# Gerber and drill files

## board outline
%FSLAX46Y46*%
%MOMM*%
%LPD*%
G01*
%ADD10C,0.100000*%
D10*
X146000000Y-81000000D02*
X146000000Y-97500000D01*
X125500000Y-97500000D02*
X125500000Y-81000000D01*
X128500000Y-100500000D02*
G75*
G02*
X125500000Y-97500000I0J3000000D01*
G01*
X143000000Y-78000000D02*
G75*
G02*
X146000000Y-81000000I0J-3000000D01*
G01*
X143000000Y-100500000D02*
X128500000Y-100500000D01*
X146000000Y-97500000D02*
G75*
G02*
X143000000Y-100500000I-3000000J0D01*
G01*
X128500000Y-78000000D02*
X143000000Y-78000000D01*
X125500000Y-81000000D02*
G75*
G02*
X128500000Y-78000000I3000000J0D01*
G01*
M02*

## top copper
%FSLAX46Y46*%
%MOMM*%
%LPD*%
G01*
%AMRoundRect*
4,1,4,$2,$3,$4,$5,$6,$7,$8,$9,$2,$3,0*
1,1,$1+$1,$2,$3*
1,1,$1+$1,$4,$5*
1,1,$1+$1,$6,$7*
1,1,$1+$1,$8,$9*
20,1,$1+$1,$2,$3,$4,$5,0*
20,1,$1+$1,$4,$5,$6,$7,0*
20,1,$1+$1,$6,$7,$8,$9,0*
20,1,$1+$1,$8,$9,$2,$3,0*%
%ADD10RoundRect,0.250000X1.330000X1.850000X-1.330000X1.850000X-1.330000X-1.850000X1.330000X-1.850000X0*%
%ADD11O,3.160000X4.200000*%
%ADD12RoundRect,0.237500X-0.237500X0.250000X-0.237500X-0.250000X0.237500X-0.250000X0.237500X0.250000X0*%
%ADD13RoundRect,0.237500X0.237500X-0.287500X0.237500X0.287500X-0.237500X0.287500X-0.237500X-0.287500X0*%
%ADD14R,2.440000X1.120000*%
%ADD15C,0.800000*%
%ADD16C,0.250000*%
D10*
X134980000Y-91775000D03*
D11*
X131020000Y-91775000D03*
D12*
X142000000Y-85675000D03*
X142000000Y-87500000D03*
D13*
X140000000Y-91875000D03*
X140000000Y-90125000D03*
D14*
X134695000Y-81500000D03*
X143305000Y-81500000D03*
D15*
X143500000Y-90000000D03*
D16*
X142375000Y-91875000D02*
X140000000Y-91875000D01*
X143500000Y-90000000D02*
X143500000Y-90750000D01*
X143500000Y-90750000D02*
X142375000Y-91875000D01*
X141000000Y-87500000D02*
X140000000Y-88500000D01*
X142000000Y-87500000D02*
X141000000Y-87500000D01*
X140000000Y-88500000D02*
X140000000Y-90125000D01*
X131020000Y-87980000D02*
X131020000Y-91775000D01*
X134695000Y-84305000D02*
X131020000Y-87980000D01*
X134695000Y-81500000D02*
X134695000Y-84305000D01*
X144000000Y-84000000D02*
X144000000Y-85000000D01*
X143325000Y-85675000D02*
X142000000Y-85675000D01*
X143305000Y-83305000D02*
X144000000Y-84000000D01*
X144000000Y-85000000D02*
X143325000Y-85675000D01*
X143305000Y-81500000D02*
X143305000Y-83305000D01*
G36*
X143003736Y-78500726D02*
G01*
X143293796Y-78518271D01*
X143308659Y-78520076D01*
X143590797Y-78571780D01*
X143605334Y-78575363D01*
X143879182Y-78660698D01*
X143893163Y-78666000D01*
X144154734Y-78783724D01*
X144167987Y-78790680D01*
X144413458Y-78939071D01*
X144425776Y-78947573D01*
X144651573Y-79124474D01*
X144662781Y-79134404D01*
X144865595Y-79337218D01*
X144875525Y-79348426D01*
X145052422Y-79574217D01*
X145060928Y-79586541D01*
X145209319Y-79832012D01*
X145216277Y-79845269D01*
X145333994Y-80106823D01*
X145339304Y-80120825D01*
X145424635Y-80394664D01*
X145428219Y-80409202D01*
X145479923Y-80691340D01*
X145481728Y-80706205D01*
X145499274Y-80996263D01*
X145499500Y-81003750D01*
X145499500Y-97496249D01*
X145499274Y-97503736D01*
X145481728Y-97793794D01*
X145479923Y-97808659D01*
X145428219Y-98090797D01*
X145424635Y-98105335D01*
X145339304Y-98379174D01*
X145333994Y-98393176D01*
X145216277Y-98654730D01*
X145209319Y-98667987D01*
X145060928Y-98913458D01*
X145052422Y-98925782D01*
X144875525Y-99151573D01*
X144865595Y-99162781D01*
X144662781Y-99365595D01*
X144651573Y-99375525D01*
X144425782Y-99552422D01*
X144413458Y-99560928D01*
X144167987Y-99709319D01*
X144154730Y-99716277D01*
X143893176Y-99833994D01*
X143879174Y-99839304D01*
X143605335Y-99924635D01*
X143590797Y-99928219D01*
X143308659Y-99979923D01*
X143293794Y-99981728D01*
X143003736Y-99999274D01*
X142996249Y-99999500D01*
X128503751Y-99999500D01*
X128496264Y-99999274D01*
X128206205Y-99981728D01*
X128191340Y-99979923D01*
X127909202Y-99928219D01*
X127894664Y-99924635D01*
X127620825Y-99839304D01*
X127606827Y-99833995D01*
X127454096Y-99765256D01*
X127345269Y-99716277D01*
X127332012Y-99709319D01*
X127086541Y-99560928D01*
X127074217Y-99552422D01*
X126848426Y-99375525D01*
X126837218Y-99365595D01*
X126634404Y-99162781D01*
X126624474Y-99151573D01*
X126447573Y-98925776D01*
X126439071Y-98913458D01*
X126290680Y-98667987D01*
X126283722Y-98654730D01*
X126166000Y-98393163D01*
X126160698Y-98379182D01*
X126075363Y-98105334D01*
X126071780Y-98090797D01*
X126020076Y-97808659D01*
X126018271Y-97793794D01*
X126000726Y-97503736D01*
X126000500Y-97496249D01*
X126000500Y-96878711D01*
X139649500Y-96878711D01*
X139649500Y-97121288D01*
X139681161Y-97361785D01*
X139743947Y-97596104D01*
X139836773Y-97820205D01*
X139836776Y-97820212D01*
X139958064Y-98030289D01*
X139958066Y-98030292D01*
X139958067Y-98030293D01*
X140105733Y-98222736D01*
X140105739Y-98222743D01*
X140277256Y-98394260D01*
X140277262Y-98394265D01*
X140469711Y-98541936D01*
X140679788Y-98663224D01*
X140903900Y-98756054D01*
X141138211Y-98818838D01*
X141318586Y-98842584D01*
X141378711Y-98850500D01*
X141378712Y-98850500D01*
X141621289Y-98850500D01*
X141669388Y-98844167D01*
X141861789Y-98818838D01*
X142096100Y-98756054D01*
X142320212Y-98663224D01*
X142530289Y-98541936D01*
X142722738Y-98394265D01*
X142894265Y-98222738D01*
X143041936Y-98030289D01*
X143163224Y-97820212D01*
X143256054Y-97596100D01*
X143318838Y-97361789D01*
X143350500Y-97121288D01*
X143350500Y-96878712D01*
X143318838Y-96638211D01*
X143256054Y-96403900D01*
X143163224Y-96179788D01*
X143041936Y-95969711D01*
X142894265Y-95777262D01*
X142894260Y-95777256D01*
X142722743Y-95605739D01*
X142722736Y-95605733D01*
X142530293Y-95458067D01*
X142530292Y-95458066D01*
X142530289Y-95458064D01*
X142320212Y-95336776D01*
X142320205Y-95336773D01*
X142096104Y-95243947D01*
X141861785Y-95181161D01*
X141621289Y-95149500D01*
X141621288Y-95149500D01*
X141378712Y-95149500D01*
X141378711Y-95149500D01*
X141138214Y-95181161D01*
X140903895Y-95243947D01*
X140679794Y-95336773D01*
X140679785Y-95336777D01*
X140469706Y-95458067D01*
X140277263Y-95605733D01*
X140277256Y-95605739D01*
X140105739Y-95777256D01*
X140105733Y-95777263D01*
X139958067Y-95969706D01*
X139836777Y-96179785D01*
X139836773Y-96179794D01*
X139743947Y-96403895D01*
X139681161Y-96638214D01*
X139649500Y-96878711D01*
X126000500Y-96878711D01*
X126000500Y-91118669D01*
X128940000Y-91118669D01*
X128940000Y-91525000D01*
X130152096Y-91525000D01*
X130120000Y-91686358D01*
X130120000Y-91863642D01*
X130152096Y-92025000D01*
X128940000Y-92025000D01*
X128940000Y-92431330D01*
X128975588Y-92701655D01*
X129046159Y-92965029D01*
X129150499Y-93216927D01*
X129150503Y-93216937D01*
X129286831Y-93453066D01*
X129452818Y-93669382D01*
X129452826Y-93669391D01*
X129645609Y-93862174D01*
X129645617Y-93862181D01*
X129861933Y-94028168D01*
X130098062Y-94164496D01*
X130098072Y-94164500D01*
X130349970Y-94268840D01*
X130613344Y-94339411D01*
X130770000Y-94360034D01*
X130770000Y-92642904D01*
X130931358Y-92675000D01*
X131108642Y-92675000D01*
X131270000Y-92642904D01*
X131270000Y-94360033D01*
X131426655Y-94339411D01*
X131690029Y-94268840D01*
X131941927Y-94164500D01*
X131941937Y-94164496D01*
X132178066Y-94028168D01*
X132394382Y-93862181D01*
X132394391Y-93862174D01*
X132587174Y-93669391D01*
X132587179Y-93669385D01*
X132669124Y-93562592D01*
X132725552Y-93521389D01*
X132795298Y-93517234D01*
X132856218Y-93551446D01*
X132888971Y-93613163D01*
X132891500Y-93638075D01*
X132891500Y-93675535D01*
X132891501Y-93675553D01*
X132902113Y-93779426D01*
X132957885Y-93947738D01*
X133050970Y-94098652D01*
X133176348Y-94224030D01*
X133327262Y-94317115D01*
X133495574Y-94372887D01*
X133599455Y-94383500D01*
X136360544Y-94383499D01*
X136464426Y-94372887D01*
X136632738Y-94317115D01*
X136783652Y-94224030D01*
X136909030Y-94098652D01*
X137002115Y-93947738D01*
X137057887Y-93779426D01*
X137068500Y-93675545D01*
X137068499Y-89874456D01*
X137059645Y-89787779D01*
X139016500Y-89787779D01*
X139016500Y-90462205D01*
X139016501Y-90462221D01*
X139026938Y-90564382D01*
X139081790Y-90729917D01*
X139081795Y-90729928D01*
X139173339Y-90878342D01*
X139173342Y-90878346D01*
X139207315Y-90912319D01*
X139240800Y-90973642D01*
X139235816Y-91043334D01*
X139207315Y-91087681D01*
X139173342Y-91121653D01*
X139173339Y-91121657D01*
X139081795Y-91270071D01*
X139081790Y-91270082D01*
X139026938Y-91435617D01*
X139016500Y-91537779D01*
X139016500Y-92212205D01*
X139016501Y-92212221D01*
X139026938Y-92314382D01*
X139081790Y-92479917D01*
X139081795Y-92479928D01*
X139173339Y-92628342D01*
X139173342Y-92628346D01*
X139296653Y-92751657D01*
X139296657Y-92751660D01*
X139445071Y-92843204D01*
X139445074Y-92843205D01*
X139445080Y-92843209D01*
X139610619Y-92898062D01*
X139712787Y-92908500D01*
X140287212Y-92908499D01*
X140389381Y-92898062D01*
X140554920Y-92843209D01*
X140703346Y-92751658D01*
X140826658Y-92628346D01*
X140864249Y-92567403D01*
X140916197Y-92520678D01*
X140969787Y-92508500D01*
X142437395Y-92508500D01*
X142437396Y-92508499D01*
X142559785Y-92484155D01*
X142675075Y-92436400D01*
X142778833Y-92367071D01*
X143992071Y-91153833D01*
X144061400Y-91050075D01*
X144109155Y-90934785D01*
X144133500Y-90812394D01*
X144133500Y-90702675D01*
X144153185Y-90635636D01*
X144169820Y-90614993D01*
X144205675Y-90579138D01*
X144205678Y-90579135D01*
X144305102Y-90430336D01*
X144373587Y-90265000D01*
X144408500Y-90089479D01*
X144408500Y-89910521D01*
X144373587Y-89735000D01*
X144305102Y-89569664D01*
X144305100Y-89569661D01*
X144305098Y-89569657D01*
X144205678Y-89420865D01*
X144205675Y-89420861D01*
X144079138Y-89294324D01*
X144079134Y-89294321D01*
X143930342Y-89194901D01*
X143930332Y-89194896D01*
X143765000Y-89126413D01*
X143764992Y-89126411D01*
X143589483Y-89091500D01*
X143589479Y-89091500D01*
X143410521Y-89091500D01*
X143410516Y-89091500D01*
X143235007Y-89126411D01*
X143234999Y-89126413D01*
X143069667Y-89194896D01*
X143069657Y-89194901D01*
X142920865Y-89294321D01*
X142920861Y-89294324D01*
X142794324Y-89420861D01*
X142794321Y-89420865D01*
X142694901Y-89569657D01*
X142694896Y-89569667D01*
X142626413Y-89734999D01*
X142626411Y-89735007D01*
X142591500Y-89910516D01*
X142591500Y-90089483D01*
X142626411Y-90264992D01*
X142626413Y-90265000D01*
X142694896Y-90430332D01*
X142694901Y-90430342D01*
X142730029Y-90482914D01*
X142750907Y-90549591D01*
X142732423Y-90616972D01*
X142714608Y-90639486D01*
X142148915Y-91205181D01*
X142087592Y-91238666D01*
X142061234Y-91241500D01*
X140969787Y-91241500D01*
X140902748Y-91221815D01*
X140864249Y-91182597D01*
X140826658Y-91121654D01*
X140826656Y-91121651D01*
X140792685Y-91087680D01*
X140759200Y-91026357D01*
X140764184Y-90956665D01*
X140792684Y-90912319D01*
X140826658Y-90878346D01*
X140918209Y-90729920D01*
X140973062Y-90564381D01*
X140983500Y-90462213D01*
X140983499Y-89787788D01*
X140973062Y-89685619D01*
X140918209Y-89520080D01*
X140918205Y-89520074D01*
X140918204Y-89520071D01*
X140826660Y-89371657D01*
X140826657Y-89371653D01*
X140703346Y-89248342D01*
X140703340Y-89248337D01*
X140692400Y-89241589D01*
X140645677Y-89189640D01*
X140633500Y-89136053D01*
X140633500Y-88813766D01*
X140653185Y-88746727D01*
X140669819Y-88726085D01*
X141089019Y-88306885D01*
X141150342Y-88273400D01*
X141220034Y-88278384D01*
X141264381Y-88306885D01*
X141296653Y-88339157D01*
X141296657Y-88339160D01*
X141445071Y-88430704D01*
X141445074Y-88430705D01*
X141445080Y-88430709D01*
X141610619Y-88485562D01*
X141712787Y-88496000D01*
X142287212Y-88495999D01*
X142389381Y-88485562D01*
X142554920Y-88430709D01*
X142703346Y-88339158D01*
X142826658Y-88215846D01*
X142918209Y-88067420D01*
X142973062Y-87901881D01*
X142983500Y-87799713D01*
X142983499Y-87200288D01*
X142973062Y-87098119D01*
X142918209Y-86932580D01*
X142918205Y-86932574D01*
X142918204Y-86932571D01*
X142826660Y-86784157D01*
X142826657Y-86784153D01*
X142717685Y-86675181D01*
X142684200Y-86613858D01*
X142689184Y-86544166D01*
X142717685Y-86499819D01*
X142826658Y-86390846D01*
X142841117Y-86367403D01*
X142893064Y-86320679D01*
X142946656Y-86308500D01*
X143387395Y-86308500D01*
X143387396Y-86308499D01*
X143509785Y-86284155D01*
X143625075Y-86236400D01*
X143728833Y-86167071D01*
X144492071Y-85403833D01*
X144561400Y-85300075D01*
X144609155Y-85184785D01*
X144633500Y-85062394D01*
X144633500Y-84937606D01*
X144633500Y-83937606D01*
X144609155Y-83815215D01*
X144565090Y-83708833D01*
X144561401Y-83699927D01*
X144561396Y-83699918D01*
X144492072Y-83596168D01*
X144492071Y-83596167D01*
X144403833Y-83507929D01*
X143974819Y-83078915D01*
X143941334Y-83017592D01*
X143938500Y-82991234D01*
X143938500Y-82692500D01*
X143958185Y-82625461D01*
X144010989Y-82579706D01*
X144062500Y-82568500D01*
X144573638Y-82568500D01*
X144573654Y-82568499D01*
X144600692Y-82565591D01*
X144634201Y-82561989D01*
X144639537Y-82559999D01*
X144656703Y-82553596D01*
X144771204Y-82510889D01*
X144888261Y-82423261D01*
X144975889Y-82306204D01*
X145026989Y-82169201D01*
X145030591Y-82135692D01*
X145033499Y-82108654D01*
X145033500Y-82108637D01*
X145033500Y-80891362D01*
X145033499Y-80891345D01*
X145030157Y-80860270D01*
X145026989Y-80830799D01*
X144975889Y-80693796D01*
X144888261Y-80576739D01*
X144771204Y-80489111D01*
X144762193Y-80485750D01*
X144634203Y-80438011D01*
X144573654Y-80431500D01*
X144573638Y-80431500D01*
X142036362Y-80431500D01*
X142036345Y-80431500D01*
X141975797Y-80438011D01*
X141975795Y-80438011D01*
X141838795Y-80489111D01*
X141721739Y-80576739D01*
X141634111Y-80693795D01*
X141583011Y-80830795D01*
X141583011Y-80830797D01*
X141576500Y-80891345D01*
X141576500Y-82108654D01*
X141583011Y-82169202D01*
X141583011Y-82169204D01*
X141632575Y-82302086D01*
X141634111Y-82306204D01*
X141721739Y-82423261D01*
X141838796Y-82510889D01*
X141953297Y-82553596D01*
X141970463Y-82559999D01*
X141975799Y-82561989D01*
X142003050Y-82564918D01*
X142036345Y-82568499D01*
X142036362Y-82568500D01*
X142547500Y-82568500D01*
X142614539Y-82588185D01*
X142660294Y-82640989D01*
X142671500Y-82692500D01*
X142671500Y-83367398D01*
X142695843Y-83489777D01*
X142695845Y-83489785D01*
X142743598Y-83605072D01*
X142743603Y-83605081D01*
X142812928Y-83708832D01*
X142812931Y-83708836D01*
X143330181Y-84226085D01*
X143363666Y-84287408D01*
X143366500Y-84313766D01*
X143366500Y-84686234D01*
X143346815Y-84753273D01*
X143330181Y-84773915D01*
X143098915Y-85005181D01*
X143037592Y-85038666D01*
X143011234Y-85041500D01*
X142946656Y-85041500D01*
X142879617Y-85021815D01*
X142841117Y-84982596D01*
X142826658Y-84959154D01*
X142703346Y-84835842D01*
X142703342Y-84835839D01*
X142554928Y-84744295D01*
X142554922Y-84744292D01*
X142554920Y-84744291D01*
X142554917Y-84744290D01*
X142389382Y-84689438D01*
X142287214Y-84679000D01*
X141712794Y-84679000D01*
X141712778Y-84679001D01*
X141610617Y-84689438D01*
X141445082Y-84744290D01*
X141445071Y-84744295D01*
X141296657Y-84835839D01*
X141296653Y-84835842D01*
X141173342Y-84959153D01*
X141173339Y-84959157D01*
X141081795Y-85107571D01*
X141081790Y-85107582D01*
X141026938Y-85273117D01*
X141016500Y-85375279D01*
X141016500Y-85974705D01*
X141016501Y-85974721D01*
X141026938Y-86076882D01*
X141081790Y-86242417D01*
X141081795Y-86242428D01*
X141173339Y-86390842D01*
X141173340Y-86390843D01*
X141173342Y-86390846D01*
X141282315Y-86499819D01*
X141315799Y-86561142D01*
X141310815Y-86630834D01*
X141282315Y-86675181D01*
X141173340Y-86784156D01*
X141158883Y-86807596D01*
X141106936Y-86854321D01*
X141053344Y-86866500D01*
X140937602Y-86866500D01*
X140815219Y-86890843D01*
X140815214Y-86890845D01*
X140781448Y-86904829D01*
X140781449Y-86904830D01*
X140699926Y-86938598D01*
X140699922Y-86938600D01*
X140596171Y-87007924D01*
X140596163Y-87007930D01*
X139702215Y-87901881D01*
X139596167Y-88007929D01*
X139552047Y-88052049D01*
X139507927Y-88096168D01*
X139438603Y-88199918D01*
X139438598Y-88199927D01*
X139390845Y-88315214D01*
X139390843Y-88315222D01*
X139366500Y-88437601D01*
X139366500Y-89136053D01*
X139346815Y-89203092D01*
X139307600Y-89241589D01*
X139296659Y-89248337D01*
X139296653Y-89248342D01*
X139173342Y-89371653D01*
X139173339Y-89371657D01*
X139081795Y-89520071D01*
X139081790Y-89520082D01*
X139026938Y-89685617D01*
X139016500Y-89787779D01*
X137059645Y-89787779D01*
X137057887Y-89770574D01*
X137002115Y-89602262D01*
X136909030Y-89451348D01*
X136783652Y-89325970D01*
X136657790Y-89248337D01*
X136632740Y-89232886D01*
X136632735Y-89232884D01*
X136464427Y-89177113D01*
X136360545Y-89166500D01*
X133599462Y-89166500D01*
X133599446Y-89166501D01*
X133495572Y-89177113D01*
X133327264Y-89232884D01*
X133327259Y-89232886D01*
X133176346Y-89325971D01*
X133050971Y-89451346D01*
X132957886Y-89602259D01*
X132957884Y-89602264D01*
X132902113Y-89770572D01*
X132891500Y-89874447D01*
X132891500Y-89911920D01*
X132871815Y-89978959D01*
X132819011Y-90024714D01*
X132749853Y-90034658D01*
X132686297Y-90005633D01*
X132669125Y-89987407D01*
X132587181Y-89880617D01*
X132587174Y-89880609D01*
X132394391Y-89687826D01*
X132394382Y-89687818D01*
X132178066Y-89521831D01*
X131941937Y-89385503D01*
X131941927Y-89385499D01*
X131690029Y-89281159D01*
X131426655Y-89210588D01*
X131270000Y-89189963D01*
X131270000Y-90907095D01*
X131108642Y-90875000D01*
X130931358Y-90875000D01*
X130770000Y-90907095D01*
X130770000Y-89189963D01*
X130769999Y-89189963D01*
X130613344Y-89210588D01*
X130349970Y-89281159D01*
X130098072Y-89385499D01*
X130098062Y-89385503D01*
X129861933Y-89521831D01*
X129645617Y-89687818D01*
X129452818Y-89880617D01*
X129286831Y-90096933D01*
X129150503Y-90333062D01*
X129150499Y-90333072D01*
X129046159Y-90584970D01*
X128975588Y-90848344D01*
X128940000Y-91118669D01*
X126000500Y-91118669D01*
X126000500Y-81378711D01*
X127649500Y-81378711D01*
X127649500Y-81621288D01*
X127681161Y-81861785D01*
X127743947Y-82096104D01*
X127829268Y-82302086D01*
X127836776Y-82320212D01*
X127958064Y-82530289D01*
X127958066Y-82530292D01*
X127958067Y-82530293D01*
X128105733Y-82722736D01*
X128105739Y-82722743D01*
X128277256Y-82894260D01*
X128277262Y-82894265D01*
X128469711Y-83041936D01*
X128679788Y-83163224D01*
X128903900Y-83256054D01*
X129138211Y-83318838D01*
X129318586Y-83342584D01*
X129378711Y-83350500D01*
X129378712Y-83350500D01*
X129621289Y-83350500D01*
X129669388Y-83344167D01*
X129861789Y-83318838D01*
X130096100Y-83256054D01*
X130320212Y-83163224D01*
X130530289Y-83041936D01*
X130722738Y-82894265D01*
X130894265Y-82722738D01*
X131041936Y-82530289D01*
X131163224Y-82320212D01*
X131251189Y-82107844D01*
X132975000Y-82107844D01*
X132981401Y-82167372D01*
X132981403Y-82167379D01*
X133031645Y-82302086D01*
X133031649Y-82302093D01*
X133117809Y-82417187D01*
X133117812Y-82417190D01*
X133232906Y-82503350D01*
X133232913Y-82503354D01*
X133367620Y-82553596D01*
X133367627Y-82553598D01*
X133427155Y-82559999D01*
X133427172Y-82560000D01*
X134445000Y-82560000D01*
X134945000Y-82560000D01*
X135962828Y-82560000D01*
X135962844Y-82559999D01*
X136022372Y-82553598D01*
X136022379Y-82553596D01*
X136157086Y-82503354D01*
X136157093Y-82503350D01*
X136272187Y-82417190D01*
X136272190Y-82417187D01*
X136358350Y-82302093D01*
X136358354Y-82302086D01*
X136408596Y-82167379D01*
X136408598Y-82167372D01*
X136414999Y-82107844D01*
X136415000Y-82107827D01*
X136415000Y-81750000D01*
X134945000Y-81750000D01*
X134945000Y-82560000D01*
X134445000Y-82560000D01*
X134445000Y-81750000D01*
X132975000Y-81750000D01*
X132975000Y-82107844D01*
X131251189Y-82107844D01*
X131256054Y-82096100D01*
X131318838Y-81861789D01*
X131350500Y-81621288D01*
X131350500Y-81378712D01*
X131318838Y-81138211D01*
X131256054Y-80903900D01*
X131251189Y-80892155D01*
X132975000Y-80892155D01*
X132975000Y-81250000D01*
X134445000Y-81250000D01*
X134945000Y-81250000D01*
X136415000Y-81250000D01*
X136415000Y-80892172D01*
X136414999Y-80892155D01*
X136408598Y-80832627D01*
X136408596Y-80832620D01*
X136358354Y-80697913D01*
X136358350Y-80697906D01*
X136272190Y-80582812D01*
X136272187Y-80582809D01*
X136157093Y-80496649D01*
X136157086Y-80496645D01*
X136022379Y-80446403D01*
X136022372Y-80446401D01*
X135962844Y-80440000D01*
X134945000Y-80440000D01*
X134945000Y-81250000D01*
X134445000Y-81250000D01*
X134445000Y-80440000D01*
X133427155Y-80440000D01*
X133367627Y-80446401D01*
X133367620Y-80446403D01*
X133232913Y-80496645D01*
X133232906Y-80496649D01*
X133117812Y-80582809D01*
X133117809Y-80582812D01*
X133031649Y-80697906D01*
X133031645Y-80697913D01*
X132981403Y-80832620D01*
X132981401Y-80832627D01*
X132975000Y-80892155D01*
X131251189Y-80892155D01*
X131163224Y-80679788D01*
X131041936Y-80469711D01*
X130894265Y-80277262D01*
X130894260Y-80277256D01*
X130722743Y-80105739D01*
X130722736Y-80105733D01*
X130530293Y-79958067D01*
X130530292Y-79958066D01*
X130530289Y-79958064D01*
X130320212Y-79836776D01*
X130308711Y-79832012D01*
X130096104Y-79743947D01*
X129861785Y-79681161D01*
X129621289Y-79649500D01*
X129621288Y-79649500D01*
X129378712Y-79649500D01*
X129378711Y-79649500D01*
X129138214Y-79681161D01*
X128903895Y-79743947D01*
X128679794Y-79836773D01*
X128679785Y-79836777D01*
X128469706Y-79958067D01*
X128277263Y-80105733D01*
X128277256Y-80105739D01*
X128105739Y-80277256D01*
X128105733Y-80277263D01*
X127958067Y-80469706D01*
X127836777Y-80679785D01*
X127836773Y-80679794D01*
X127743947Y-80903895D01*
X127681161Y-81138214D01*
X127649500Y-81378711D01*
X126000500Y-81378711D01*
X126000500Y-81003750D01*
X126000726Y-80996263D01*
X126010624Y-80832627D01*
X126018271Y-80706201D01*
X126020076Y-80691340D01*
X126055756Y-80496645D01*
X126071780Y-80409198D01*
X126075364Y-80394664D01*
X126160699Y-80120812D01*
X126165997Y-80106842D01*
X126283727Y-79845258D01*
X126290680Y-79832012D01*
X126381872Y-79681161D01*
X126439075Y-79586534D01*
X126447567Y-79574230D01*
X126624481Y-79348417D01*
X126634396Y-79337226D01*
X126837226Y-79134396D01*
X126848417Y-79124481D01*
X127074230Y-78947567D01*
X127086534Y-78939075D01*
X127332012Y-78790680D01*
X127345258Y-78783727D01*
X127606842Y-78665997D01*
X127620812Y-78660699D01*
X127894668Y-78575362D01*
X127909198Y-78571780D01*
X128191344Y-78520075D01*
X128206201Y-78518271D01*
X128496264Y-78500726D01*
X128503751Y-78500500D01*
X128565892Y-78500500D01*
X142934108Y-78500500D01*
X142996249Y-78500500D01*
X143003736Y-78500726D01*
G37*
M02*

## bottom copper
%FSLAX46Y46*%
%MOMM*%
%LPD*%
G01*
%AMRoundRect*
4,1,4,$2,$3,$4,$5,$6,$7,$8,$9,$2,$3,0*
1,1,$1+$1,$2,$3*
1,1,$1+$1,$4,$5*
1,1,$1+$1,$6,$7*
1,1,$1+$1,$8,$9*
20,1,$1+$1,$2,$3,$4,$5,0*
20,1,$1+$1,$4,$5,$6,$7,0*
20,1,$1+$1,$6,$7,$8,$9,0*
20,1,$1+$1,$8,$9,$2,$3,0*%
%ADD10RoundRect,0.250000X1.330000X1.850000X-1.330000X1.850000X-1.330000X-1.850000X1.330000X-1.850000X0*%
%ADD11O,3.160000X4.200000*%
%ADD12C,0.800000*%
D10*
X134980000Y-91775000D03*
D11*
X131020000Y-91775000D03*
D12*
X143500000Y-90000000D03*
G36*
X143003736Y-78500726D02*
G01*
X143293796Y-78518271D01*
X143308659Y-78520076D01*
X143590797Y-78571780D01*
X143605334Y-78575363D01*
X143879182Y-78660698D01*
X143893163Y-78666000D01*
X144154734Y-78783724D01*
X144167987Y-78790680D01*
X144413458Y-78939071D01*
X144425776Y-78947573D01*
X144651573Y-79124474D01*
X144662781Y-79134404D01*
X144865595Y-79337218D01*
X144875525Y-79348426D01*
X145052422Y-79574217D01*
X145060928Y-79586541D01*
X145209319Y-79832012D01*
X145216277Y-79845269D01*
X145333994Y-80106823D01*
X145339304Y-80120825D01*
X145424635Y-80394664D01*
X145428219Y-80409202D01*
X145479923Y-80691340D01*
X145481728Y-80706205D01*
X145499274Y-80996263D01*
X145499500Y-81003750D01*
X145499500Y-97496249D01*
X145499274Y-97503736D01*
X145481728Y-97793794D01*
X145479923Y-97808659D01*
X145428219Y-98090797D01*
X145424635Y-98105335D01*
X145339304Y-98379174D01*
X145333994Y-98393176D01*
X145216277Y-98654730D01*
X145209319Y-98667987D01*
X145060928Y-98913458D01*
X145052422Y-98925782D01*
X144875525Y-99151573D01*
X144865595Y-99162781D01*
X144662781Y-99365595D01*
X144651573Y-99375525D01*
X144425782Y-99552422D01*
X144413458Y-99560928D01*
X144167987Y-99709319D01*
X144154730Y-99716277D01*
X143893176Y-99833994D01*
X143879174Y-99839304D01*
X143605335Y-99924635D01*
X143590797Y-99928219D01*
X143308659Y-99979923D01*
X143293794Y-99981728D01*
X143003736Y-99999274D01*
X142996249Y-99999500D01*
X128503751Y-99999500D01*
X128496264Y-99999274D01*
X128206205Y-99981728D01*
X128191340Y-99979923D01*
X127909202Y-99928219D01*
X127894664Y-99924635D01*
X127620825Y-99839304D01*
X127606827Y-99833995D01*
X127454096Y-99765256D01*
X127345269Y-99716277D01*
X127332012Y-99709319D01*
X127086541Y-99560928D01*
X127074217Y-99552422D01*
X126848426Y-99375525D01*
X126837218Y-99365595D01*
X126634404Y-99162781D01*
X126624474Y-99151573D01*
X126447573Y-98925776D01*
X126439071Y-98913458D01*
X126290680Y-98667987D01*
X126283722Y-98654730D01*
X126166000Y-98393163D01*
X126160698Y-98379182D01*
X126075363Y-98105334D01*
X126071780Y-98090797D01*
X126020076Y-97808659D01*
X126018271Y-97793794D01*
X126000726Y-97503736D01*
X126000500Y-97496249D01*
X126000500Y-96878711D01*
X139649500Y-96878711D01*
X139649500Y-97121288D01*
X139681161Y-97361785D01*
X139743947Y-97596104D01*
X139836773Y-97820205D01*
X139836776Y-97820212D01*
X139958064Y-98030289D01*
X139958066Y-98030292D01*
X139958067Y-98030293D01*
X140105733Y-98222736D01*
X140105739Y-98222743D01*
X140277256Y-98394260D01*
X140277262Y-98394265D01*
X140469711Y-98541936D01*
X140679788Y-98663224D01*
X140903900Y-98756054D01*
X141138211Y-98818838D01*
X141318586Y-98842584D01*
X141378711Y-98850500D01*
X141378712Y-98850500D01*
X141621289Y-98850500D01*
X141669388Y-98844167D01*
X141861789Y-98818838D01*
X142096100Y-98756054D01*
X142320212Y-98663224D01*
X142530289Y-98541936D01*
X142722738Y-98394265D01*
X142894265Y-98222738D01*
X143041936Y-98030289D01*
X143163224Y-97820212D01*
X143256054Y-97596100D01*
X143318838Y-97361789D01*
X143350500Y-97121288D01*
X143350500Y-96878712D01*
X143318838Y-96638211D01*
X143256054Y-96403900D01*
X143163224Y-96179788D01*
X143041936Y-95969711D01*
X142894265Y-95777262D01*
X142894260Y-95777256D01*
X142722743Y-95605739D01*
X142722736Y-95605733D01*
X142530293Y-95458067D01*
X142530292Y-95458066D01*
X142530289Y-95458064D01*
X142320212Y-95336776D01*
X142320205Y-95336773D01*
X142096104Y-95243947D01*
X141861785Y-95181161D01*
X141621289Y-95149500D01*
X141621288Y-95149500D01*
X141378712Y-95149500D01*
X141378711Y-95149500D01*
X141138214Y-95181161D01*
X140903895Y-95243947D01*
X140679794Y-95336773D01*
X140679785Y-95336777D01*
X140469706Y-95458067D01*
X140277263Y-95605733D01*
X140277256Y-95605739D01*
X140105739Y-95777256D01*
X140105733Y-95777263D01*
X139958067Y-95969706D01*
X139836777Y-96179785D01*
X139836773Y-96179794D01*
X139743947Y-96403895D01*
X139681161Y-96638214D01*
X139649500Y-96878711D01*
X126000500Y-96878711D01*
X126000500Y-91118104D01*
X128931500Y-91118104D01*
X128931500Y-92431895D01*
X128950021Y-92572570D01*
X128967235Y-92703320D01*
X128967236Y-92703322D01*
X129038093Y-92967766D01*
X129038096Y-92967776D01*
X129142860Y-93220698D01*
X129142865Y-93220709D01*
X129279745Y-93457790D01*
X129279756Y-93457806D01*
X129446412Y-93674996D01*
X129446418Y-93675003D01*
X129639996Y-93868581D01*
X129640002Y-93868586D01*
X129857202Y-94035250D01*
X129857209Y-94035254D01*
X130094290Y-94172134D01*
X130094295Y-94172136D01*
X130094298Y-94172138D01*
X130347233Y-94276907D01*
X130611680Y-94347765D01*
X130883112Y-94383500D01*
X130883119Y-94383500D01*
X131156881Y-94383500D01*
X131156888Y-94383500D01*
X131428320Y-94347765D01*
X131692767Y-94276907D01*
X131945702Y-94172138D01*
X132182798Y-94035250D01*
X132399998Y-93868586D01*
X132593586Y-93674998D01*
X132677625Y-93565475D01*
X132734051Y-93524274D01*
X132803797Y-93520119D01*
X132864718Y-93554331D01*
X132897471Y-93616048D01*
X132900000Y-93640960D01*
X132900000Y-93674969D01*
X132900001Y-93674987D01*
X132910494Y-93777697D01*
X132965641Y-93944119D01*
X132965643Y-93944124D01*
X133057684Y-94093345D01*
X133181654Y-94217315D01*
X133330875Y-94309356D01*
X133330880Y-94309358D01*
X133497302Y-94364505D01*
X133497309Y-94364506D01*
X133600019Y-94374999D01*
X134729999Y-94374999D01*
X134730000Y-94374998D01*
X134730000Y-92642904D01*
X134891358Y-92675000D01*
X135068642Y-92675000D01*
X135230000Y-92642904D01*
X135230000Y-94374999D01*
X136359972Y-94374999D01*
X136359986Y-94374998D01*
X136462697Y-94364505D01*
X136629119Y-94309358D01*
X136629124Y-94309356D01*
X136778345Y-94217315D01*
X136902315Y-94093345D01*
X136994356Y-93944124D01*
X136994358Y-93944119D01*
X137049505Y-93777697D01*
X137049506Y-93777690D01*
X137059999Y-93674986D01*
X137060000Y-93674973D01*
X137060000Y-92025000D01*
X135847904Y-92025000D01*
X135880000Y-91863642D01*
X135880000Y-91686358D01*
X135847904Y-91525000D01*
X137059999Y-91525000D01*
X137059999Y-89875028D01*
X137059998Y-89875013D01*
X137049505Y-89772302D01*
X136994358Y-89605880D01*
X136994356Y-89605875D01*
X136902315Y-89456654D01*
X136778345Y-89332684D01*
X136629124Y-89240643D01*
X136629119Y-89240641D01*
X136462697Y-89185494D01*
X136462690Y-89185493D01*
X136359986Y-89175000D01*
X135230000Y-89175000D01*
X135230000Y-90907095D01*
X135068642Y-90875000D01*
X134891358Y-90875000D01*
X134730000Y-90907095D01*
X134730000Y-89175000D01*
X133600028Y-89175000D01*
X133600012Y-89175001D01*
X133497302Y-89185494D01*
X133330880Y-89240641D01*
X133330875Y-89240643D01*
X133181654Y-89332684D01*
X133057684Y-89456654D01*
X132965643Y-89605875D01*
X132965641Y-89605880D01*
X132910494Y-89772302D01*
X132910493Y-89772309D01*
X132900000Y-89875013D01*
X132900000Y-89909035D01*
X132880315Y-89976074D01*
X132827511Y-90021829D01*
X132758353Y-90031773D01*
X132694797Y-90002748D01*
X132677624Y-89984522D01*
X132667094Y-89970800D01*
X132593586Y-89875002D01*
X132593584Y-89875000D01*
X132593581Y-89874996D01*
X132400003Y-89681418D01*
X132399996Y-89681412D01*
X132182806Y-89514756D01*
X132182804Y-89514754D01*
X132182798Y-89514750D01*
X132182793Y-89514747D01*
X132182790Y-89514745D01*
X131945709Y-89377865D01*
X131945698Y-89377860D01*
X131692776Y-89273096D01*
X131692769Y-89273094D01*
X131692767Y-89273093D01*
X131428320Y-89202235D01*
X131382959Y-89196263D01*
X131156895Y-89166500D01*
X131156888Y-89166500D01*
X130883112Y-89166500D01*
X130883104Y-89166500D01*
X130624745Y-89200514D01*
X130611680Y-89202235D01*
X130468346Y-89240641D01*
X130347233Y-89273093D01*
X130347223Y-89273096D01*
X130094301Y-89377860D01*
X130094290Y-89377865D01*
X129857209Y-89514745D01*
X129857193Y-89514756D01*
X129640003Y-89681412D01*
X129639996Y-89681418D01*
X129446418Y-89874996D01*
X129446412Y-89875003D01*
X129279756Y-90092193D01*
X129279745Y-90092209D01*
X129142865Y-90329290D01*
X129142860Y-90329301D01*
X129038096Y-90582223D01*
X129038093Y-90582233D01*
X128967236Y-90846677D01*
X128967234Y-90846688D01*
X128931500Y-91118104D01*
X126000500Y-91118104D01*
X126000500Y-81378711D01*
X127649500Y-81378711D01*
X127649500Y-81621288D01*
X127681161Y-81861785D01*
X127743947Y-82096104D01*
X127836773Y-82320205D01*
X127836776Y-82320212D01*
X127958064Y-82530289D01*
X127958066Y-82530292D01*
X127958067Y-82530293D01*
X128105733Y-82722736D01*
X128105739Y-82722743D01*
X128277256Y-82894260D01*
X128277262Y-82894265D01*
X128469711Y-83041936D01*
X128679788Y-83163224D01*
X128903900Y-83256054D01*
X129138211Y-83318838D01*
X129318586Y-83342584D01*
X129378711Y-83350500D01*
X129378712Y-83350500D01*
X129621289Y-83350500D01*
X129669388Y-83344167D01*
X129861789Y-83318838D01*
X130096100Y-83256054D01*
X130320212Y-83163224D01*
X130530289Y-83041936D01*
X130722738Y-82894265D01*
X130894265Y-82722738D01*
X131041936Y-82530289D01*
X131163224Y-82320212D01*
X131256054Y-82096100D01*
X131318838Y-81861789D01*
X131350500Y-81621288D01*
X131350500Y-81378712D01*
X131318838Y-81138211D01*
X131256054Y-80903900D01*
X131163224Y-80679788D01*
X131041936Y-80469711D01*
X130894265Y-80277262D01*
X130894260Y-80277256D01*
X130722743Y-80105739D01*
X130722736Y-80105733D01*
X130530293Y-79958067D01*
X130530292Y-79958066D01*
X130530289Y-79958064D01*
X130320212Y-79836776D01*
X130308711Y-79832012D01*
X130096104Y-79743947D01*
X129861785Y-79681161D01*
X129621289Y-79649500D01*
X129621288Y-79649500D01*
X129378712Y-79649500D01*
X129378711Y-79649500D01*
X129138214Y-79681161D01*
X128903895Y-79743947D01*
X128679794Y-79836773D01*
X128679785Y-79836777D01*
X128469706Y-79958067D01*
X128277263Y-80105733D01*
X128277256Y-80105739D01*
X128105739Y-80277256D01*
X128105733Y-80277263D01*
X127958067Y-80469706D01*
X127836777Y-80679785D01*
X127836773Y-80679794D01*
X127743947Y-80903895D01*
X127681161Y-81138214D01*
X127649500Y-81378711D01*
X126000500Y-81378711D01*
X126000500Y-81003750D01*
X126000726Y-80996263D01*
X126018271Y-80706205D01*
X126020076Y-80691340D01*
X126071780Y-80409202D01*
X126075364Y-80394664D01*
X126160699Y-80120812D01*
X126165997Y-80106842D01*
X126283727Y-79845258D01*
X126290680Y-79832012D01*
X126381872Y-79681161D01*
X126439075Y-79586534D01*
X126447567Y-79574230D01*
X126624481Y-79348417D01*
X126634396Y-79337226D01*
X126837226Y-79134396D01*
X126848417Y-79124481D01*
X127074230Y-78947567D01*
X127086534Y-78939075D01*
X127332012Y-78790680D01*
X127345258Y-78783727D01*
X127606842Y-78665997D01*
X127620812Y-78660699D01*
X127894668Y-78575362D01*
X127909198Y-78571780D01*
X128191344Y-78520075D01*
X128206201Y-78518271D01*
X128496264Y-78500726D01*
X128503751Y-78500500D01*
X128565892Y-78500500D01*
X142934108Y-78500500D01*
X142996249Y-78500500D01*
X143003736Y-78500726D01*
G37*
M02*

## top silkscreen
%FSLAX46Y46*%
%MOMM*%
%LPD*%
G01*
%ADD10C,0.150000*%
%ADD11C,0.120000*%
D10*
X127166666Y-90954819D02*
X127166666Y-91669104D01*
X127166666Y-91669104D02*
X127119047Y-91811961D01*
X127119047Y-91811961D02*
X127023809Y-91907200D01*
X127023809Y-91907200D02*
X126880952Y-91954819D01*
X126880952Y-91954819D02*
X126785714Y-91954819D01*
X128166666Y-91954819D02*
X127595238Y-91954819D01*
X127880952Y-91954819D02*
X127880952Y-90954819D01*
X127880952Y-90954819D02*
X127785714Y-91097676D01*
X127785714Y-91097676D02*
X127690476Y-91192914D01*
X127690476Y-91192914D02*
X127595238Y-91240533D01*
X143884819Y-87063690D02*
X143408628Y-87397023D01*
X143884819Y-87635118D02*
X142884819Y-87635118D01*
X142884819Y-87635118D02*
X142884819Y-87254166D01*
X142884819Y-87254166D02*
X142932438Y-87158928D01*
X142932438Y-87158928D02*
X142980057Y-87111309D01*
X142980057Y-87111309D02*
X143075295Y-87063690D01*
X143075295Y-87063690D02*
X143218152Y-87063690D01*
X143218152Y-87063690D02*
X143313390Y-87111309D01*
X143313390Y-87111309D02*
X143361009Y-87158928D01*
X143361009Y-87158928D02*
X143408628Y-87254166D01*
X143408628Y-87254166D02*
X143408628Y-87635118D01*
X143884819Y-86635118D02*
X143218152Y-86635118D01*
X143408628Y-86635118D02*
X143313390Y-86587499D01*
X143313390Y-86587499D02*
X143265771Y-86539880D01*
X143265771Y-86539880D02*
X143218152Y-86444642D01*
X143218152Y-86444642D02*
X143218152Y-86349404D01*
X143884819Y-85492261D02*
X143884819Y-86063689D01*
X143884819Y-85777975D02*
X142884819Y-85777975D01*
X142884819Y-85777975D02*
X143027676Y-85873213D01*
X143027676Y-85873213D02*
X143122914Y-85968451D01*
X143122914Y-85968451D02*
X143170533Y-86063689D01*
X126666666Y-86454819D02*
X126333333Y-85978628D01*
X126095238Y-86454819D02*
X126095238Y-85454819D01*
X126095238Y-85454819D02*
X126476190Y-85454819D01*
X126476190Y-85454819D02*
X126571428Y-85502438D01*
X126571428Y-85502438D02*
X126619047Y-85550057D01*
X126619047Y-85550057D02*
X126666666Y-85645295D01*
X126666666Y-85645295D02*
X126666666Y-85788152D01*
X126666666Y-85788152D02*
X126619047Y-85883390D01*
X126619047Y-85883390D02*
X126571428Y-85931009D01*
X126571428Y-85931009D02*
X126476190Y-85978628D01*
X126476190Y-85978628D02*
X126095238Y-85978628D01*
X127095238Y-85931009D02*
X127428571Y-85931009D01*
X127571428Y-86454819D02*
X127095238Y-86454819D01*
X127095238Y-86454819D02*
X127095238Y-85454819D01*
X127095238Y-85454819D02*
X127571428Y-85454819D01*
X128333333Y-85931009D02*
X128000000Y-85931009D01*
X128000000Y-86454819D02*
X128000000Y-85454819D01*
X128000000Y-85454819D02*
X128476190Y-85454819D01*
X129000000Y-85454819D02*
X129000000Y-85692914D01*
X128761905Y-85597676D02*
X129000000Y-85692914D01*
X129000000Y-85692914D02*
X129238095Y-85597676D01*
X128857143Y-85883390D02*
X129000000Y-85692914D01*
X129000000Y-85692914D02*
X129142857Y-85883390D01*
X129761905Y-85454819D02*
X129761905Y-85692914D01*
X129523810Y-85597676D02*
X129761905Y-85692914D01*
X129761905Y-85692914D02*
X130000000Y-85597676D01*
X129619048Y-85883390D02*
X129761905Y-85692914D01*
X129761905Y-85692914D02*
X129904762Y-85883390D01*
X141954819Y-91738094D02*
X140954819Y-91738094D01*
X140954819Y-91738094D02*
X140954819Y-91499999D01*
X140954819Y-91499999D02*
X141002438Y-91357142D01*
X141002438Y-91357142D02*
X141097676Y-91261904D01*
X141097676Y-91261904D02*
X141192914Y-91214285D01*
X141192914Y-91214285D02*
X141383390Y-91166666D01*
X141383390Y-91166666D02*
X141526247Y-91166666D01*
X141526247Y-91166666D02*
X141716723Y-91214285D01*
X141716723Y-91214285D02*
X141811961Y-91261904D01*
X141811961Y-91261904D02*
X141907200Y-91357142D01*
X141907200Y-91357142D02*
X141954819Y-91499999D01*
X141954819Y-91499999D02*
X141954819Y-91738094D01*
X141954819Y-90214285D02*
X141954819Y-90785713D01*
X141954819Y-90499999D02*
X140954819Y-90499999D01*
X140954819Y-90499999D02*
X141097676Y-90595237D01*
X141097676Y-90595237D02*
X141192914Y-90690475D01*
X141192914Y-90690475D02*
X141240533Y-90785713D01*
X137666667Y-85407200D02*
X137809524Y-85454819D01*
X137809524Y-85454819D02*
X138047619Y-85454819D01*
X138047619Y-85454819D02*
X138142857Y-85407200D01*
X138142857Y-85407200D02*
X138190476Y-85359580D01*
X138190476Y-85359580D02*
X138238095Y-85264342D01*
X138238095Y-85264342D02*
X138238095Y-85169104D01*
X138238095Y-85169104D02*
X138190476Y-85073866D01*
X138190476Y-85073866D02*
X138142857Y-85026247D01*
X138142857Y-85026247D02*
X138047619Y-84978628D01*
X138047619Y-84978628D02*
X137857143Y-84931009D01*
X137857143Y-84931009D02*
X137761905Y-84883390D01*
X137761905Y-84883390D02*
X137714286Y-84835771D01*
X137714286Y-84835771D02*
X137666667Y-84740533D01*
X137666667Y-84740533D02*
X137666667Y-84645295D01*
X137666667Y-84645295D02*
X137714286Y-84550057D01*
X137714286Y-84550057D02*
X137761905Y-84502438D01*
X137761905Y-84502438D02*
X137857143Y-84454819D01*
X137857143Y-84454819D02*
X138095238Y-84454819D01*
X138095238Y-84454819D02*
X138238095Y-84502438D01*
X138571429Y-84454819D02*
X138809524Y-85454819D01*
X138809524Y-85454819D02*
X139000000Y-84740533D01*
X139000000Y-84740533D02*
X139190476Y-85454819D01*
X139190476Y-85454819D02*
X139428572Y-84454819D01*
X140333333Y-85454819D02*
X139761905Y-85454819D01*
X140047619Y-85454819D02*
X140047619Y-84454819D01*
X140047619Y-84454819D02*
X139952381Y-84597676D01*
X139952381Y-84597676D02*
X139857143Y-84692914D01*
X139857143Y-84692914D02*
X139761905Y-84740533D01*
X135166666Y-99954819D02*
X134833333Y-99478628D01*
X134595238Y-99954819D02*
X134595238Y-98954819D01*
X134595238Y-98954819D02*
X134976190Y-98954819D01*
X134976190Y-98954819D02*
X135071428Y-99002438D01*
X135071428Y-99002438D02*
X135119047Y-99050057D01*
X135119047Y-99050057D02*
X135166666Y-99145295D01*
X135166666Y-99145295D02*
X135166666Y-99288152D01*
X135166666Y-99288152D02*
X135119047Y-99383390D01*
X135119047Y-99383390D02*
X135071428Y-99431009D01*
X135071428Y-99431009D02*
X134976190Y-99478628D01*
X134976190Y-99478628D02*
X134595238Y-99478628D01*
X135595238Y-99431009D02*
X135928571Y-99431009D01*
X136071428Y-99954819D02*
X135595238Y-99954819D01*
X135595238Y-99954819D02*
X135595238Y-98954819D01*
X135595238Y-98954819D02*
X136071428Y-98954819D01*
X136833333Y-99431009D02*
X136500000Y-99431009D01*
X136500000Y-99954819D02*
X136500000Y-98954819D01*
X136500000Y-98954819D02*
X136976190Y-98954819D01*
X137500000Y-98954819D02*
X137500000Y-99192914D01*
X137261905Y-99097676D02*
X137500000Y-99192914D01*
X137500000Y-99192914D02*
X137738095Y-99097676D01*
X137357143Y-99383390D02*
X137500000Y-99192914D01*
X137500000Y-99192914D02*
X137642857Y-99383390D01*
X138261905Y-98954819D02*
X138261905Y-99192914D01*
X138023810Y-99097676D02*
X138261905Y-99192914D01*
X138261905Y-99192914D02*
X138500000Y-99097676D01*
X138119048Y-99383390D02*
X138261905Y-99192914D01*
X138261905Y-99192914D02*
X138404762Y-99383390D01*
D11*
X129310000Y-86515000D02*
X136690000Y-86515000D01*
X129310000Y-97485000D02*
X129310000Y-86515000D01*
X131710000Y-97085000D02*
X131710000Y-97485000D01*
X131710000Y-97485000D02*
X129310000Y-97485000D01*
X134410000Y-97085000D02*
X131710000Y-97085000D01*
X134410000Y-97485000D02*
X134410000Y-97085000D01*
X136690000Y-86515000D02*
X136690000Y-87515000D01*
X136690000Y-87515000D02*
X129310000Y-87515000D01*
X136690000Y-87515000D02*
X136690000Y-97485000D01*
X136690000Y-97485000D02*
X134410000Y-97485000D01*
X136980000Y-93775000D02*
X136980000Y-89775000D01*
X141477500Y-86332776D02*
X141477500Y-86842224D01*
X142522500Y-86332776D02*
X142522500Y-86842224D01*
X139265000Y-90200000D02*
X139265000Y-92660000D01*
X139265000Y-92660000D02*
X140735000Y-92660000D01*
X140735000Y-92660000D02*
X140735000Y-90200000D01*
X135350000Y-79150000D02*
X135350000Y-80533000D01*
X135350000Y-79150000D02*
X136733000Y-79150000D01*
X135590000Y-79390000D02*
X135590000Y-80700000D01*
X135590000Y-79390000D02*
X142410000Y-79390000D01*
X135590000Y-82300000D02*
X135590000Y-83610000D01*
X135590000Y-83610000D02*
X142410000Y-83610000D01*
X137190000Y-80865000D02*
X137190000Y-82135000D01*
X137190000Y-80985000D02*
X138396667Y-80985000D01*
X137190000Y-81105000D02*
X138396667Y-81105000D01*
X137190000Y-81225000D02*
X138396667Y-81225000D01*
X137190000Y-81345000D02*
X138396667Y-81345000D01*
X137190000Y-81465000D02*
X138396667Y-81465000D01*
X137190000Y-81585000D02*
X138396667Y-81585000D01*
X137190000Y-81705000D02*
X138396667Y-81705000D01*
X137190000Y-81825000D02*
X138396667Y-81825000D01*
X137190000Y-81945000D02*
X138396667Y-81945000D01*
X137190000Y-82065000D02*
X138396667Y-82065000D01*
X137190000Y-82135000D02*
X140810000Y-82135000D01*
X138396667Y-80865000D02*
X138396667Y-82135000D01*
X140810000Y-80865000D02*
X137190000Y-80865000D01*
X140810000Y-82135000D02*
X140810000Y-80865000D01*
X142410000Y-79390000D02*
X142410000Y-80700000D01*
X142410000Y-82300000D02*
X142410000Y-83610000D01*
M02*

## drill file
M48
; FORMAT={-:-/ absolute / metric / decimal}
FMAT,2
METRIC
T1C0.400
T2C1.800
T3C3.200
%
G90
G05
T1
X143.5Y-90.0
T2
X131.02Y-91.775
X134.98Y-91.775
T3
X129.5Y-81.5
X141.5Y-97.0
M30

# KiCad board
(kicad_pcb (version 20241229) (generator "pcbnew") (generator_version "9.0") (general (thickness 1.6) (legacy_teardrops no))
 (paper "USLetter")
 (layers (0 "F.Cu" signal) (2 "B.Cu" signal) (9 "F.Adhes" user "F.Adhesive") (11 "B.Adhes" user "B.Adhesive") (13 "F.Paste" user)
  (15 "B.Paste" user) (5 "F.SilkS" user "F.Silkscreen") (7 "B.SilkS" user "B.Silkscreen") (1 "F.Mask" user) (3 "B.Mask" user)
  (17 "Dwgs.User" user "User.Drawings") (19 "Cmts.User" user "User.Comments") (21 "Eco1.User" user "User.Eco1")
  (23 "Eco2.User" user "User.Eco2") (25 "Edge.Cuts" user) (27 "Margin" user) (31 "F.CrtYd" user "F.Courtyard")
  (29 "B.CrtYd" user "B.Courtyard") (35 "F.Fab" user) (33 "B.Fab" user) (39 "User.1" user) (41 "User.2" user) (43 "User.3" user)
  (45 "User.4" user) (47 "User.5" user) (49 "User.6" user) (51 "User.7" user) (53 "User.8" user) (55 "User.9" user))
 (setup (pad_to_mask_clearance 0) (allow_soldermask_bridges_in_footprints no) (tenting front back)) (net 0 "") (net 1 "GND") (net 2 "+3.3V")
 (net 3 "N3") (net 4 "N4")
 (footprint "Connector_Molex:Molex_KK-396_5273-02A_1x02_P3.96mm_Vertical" (layer "F.Cu") (at 134.98 91.775 180)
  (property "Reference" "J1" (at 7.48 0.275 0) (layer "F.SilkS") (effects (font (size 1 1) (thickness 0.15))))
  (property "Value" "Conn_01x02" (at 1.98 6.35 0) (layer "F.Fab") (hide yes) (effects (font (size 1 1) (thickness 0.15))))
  (fp_line (start 5.67 5.26) (end -1.71 5.26) (stroke (width 0.12) (type solid)) (layer "F.SilkS"))
  (fp_line (start 5.67 -5.71) (end 5.67 5.26) (stroke (width 0.12) (type solid)) (layer "F.SilkS"))
  (fp_line (start 3.27 -5.31) (end 3.27 -5.71) (stroke (width 0.12) (type solid)) (layer "F.SilkS"))
  (fp_line (start 3.27 -5.71) (end 5.67 -5.71) (stroke (width 0.12) (type solid)) (layer "F.SilkS"))
  (fp_line (start 0.57 -5.31) (end 3.27 -5.31) (stroke (width 0.12) (type solid)) (layer "F.SilkS"))
  (fp_line (start 0.57 -5.71) (end 0.57 -5.31) (stroke (width 0.12) (type solid)) (layer "F.SilkS"))
  (fp_line (start -1.71 5.26) (end -1.71 4.26) (stroke (width 0.12) (type solid)) (layer "F.SilkS"))
  (fp_line (start -1.71 4.26) (end 5.67 4.26) (stroke (width 0.12) (type solid)) (layer "F.SilkS"))
  (fp_line (start -1.71 4.26) (end -1.71 -5.71) (stroke (width 0.12) (type solid)) (layer "F.SilkS"))
  (fp_line (start -1.71 -5.71) (end 0.57 -5.71) (stroke (width 0.12) (type solid)) (layer "F.SilkS"))
  (fp_line (start -2 -2) (end -2 2) (stroke (width 0.12) (type solid)) (layer "F.SilkS"))
  (pad "1" thru_hole roundrect (at 0 0 180) (size 3.16 4.2) (drill 1.8) (layers "*.Cu" "*.Mask") (remove_unused_layers no)
   (roundrect_rratio 0.079114) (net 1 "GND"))
  (pad "2" thru_hole oval (at 3.96 0 180) (size 3.16 4.2) (drill 1.8) (layers "*.Cu" "*.Mask") (remove_unused_layers no) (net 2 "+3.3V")))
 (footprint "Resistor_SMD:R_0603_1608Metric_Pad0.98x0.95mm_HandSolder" (layer "F.Cu") (at 142 86.5875 -90)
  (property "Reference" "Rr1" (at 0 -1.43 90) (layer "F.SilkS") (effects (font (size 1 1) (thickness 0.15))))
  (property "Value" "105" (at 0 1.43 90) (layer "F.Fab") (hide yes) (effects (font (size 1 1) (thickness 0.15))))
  (fp_line (start -0.254724 0.5225) (end 0.254724 0.5225) (stroke (width 0.12) (type solid)) (layer "F.SilkS"))
  (fp_line (start -0.254724 -0.5225) (end 0.254724 -0.5225) (stroke (width 0.12) (type solid)) (layer "F.SilkS"))
  (pad "1" smd roundrect (at -0.9125 0 270) (size 0.975 0.95) (layers "F.Cu" "F.Mask" "F.Paste") (roundrect_rratio 0.25) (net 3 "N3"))
  (pad "2" smd roundrect (at 0.9125 0 270) (size 0.975 0.95) (layers "F.Cu" "F.Mask" "F.Paste") (roundrect_rratio 0.25) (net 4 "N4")))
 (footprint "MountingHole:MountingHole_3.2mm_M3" (layer "F.Cu") (at 129.5 81.5)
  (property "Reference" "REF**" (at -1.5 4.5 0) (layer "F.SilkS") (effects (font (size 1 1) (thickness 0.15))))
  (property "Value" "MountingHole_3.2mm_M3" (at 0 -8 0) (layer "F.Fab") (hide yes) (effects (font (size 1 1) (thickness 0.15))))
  (pad "" np_thru_hole circle (at 0 0) (size 3.2 3.2) (drill 3.2) (layers "*.Cu" "*.Mask")))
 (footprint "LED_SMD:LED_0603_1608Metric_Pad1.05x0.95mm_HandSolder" (layer "F.Cu") (at 140 91 90)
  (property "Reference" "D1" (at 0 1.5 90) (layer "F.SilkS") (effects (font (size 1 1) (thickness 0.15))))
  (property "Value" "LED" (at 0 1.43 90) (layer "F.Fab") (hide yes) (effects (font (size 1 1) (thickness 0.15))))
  (fp_line (start 0.8 -0.735) (end -1.66 -0.735) (stroke (width 0.12) (type solid)) (layer "F.SilkS"))
  (fp_line (start -1.66 -0.735) (end -1.66 0.735) (stroke (width 0.12) (type solid)) (layer "F.SilkS"))
  (fp_line (start -1.66 0.735) (end 0.8 0.735) (stroke (width 0.12) (type solid)) (layer "F.SilkS"))
  (pad "1" smd roundrect (at -0.875 0 90) (size 1.05 0.95) (layers "F.Cu" "F.Mask" "F.Paste") (roundrect_rratio 0.25) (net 1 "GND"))
  (pad "2" smd roundrect (at 0.875 0 90) (size 1.05 0.95) (layers "F.Cu" "F.Mask" "F.Paste") (roundrect_rratio 0.25) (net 4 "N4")))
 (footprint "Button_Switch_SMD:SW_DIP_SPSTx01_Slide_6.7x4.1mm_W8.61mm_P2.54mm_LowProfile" (layer "F.Cu") (at 139 81.5)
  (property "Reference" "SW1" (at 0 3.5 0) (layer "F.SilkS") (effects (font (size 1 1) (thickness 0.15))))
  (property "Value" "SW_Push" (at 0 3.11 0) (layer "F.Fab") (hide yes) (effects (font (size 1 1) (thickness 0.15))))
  (fp_line (start -3.65 -2.35) (end -3.65 -0.967) (stroke (width 0.12) (type solid)) (layer "F.SilkS"))
  (fp_line (start -3.65 -2.35) (end -2.267 -2.35) (stroke (width 0.12) (type solid)) (layer "F.SilkS"))
  (fp_line (start -3.41 -2.11) (end -3.41 -0.8) (stroke (width 0.12) (type solid)) (layer "F.SilkS"))
  (fp_line (start -3.41 -2.11) (end 3.41 -2.11) (stroke (width 0.12) (type solid)) (layer "F.SilkS"))
  (fp_line (start -3.41 0.8) (end -3.41 2.11) (stroke (width 0.12) (type solid)) (layer "F.SilkS"))
  (fp_line (start -3.41 2.11) (end 3.41 2.11) (stroke (width 0.12) (type solid)) (layer "F.SilkS"))
  (fp_line (start -1.81 -0.635) (end -1.81 0.635) (stroke (width 0.12) (type solid)) (layer "F.SilkS"))
  (fp_line (start -1.81 -0.515) (end -0.603333 -0.515) (stroke (width 0.12) (type solid)) (layer "F.SilkS"))
  (fp_line (start -1.81 -0.395) (end -0.603333 -0.395) (stroke (width 0.12) (type solid)) (layer "F.SilkS"))
  (fp_line (start -1.81 -0.275) (end -0.603333 -0.275) (stroke (width 0.12) (type solid)) (layer "F.SilkS"))
  (fp_line (start -1.81 -0.155) (end -0.603333 -0.155) (stroke (width 0.12) (type solid)) (layer "F.SilkS"))
  (fp_line (start -1.81 -0.035) (end -0.603333 -0.035) (stroke (width 0.12) (type solid)) (layer "F.SilkS"))
  (fp_line (start -1.81 0.085) (end -0.603333 0.085) (stroke (width 0.12) (type solid)) (layer "F.SilkS"))
  (fp_line (start -1.81 0.205) (end -0.603333 0.205) (stroke (width 0.12) (type solid)) (layer "F.SilkS"))
  (fp_line (start -1.81 0.325) (end -0.603333 0.325) (stroke (width 0.12) (type solid)) (layer "F.SilkS"))
  (fp_line (start -1.81 0.445) (end -0.603333 0.445) (stroke (width 0.12) (type solid)) (layer "F.SilkS"))
  (fp_line (start -1.81 0.565) (end -0.603333 0.565) (stroke (width 0.12) (type solid)) (layer "F.SilkS"))
  (fp_line (start -1.81 0.635) (end 1.81 0.635) (stroke (width 0.12) (type solid)) (layer "F.SilkS"))
  (fp_line (start -0.603333 -0.635) (end -0.603333 0.635) (stroke (width 0.12) (type solid)) (layer "F.SilkS"))
  (fp_line (start 1.81 -0.635) (end -1.81 -0.635) (stroke (width 0.12) (type solid)) (layer "F.SilkS"))
  (fp_line (start 1.81 0.635) (end 1.81 -0.635) (stroke (width 0.12) (type solid)) (layer "F.SilkS"))
  (fp_line (start 3.41 -2.11) (end 3.41 -0.8) (stroke (width 0.12) (type solid)) (layer "F.SilkS"))
  (fp_line (start 3.41 0.8) (end 3.41 2.11) (stroke (width 0.12) (type solid)) (layer "F.SilkS"))
  (pad "1" smd rect (at -4.305 0) (size 2.44 1.12) (layers "F.Cu" "F.Mask" "F.Paste") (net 2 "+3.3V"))
  (pad "2" smd rect (at 4.305 0) (size 2.44 1.12) (layers "F.Cu" "F.Mask" "F.Paste") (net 3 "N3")))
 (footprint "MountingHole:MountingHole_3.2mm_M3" (layer "F.Cu") (at 141.5 97)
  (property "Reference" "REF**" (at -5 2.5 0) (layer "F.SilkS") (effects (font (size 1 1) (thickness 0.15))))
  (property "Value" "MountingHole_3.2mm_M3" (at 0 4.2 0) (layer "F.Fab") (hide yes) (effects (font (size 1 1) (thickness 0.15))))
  (pad "" np_thru_hole circle (at 0 0) (size 3.2 3.2) (drill 3.2) (layers "*.Cu" "*.Mask")))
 (gr_line (start 146 81) (end 146 97.5) (stroke (width 0.1) (type default)) (layer "Edge.Cuts"))
 (gr_line (start 125.5 97.5) (end 125.5 81) (stroke (width 0.1) (type default)) (layer "Edge.Cuts"))
 (gr_arc (start 128.5 100.5) (mid 126.37868 99.62132) (end 125.5 97.5) (stroke (width 0.1) (type default)) (layer "Edge.Cuts"))
 (gr_arc (start 143 78) (mid 145.12132 78.87868) (end 146 81) (stroke (width 0.1) (type default)) (layer "Edge.Cuts"))
 (gr_line (start 143 100.5) (end 128.5 100.5) (stroke (width 0.1) (type default)) (layer "Edge.Cuts"))
 (gr_arc (start 146 97.5) (mid 145.12132 99.62132) (end 143 100.5) (stroke (width 0.1) (type default)) (layer "Edge.Cuts"))
 (gr_line (start 128.5 78) (end 143 78) (stroke (width 0.1) (type default)) (layer "Edge.Cuts"))
 (gr_arc (start 125.5 81) (mid 126.37868 78.87868) (end 128.5 78) (stroke (width 0.1) (type default)) (layer "Edge.Cuts"))
 (segment (start 142.375 91.875) (end 140 91.875) (width 0.25) (layer "F.Cu") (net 1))
 (segment (start 143.5 90) (end 143.5 90.75) (width 0.25) (layer "F.Cu") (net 1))
 (segment (start 143.5 90.75) (end 142.375 91.875) (width 0.25) (layer "F.Cu") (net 1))
 (via (at 143.5 90) (size 0.8) (drill 0.4) (layers "F.Cu" "B.Cu") (free yes) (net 1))
 (segment (start 141 87.5) (end 140 88.5) (width 0.25) (layer "F.Cu") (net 4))
 (segment (start 142 87.5) (end 141 87.5) (width 0.25) (layer "F.Cu") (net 4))
 (segment (start 140 88.5) (end 140 90.125) (width 0.25) (layer "F.Cu") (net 4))
 (segment (start 131.02 87.98) (end 131.02 91.775) (width 0.25) (layer "F.Cu") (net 2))
 (segment (start 134.695 84.305) (end 131.02 87.98) (width 0.25) (layer "F.Cu") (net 2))
 (segment (start 134.695 81.5) (end 134.695 84.305) (width 0.25) (layer "F.Cu") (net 2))
 (segment (start 144 84) (end 144 85) (width 0.25) (layer "F.Cu") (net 3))
 (segment (start 143.325 85.675) (end 142 85.675) (width 0.25) (layer "F.Cu") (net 3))
 (segment (start 143.305 83.305) (end 144 84) (width 0.25) (layer "F.Cu") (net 3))
 (segment (start 144 85) (end 143.325 85.675) (width 0.25) (layer "F.Cu") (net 3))
 (segment (start 143.305 81.5) (end 143.305 83.305) (width 0.25) (layer "F.Cu") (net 3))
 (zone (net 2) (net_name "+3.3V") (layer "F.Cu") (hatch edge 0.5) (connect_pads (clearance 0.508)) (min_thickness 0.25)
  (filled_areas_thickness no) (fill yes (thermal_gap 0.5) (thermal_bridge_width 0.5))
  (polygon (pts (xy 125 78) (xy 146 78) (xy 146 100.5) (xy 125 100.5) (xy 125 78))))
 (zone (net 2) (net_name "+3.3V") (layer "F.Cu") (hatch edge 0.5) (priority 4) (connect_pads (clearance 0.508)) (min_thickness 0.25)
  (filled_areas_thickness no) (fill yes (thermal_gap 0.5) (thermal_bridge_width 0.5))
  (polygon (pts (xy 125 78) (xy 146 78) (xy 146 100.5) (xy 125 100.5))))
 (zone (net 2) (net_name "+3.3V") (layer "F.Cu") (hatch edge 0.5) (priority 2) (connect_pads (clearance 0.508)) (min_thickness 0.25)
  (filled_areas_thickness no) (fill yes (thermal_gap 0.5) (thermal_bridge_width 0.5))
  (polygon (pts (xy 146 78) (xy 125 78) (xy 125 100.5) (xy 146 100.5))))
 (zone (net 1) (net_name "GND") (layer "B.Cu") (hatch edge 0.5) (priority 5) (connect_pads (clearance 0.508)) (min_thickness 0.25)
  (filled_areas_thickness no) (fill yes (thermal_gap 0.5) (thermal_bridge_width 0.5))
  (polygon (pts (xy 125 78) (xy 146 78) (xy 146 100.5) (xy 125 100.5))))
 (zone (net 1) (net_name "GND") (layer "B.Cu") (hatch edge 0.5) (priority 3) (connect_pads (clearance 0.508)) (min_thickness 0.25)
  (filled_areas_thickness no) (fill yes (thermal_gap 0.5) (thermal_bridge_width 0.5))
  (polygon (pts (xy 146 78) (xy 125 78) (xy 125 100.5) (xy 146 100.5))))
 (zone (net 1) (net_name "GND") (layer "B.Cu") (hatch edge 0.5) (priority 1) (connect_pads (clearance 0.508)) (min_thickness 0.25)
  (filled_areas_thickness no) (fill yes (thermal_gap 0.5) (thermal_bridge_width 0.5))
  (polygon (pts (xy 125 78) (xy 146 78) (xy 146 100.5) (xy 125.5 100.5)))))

